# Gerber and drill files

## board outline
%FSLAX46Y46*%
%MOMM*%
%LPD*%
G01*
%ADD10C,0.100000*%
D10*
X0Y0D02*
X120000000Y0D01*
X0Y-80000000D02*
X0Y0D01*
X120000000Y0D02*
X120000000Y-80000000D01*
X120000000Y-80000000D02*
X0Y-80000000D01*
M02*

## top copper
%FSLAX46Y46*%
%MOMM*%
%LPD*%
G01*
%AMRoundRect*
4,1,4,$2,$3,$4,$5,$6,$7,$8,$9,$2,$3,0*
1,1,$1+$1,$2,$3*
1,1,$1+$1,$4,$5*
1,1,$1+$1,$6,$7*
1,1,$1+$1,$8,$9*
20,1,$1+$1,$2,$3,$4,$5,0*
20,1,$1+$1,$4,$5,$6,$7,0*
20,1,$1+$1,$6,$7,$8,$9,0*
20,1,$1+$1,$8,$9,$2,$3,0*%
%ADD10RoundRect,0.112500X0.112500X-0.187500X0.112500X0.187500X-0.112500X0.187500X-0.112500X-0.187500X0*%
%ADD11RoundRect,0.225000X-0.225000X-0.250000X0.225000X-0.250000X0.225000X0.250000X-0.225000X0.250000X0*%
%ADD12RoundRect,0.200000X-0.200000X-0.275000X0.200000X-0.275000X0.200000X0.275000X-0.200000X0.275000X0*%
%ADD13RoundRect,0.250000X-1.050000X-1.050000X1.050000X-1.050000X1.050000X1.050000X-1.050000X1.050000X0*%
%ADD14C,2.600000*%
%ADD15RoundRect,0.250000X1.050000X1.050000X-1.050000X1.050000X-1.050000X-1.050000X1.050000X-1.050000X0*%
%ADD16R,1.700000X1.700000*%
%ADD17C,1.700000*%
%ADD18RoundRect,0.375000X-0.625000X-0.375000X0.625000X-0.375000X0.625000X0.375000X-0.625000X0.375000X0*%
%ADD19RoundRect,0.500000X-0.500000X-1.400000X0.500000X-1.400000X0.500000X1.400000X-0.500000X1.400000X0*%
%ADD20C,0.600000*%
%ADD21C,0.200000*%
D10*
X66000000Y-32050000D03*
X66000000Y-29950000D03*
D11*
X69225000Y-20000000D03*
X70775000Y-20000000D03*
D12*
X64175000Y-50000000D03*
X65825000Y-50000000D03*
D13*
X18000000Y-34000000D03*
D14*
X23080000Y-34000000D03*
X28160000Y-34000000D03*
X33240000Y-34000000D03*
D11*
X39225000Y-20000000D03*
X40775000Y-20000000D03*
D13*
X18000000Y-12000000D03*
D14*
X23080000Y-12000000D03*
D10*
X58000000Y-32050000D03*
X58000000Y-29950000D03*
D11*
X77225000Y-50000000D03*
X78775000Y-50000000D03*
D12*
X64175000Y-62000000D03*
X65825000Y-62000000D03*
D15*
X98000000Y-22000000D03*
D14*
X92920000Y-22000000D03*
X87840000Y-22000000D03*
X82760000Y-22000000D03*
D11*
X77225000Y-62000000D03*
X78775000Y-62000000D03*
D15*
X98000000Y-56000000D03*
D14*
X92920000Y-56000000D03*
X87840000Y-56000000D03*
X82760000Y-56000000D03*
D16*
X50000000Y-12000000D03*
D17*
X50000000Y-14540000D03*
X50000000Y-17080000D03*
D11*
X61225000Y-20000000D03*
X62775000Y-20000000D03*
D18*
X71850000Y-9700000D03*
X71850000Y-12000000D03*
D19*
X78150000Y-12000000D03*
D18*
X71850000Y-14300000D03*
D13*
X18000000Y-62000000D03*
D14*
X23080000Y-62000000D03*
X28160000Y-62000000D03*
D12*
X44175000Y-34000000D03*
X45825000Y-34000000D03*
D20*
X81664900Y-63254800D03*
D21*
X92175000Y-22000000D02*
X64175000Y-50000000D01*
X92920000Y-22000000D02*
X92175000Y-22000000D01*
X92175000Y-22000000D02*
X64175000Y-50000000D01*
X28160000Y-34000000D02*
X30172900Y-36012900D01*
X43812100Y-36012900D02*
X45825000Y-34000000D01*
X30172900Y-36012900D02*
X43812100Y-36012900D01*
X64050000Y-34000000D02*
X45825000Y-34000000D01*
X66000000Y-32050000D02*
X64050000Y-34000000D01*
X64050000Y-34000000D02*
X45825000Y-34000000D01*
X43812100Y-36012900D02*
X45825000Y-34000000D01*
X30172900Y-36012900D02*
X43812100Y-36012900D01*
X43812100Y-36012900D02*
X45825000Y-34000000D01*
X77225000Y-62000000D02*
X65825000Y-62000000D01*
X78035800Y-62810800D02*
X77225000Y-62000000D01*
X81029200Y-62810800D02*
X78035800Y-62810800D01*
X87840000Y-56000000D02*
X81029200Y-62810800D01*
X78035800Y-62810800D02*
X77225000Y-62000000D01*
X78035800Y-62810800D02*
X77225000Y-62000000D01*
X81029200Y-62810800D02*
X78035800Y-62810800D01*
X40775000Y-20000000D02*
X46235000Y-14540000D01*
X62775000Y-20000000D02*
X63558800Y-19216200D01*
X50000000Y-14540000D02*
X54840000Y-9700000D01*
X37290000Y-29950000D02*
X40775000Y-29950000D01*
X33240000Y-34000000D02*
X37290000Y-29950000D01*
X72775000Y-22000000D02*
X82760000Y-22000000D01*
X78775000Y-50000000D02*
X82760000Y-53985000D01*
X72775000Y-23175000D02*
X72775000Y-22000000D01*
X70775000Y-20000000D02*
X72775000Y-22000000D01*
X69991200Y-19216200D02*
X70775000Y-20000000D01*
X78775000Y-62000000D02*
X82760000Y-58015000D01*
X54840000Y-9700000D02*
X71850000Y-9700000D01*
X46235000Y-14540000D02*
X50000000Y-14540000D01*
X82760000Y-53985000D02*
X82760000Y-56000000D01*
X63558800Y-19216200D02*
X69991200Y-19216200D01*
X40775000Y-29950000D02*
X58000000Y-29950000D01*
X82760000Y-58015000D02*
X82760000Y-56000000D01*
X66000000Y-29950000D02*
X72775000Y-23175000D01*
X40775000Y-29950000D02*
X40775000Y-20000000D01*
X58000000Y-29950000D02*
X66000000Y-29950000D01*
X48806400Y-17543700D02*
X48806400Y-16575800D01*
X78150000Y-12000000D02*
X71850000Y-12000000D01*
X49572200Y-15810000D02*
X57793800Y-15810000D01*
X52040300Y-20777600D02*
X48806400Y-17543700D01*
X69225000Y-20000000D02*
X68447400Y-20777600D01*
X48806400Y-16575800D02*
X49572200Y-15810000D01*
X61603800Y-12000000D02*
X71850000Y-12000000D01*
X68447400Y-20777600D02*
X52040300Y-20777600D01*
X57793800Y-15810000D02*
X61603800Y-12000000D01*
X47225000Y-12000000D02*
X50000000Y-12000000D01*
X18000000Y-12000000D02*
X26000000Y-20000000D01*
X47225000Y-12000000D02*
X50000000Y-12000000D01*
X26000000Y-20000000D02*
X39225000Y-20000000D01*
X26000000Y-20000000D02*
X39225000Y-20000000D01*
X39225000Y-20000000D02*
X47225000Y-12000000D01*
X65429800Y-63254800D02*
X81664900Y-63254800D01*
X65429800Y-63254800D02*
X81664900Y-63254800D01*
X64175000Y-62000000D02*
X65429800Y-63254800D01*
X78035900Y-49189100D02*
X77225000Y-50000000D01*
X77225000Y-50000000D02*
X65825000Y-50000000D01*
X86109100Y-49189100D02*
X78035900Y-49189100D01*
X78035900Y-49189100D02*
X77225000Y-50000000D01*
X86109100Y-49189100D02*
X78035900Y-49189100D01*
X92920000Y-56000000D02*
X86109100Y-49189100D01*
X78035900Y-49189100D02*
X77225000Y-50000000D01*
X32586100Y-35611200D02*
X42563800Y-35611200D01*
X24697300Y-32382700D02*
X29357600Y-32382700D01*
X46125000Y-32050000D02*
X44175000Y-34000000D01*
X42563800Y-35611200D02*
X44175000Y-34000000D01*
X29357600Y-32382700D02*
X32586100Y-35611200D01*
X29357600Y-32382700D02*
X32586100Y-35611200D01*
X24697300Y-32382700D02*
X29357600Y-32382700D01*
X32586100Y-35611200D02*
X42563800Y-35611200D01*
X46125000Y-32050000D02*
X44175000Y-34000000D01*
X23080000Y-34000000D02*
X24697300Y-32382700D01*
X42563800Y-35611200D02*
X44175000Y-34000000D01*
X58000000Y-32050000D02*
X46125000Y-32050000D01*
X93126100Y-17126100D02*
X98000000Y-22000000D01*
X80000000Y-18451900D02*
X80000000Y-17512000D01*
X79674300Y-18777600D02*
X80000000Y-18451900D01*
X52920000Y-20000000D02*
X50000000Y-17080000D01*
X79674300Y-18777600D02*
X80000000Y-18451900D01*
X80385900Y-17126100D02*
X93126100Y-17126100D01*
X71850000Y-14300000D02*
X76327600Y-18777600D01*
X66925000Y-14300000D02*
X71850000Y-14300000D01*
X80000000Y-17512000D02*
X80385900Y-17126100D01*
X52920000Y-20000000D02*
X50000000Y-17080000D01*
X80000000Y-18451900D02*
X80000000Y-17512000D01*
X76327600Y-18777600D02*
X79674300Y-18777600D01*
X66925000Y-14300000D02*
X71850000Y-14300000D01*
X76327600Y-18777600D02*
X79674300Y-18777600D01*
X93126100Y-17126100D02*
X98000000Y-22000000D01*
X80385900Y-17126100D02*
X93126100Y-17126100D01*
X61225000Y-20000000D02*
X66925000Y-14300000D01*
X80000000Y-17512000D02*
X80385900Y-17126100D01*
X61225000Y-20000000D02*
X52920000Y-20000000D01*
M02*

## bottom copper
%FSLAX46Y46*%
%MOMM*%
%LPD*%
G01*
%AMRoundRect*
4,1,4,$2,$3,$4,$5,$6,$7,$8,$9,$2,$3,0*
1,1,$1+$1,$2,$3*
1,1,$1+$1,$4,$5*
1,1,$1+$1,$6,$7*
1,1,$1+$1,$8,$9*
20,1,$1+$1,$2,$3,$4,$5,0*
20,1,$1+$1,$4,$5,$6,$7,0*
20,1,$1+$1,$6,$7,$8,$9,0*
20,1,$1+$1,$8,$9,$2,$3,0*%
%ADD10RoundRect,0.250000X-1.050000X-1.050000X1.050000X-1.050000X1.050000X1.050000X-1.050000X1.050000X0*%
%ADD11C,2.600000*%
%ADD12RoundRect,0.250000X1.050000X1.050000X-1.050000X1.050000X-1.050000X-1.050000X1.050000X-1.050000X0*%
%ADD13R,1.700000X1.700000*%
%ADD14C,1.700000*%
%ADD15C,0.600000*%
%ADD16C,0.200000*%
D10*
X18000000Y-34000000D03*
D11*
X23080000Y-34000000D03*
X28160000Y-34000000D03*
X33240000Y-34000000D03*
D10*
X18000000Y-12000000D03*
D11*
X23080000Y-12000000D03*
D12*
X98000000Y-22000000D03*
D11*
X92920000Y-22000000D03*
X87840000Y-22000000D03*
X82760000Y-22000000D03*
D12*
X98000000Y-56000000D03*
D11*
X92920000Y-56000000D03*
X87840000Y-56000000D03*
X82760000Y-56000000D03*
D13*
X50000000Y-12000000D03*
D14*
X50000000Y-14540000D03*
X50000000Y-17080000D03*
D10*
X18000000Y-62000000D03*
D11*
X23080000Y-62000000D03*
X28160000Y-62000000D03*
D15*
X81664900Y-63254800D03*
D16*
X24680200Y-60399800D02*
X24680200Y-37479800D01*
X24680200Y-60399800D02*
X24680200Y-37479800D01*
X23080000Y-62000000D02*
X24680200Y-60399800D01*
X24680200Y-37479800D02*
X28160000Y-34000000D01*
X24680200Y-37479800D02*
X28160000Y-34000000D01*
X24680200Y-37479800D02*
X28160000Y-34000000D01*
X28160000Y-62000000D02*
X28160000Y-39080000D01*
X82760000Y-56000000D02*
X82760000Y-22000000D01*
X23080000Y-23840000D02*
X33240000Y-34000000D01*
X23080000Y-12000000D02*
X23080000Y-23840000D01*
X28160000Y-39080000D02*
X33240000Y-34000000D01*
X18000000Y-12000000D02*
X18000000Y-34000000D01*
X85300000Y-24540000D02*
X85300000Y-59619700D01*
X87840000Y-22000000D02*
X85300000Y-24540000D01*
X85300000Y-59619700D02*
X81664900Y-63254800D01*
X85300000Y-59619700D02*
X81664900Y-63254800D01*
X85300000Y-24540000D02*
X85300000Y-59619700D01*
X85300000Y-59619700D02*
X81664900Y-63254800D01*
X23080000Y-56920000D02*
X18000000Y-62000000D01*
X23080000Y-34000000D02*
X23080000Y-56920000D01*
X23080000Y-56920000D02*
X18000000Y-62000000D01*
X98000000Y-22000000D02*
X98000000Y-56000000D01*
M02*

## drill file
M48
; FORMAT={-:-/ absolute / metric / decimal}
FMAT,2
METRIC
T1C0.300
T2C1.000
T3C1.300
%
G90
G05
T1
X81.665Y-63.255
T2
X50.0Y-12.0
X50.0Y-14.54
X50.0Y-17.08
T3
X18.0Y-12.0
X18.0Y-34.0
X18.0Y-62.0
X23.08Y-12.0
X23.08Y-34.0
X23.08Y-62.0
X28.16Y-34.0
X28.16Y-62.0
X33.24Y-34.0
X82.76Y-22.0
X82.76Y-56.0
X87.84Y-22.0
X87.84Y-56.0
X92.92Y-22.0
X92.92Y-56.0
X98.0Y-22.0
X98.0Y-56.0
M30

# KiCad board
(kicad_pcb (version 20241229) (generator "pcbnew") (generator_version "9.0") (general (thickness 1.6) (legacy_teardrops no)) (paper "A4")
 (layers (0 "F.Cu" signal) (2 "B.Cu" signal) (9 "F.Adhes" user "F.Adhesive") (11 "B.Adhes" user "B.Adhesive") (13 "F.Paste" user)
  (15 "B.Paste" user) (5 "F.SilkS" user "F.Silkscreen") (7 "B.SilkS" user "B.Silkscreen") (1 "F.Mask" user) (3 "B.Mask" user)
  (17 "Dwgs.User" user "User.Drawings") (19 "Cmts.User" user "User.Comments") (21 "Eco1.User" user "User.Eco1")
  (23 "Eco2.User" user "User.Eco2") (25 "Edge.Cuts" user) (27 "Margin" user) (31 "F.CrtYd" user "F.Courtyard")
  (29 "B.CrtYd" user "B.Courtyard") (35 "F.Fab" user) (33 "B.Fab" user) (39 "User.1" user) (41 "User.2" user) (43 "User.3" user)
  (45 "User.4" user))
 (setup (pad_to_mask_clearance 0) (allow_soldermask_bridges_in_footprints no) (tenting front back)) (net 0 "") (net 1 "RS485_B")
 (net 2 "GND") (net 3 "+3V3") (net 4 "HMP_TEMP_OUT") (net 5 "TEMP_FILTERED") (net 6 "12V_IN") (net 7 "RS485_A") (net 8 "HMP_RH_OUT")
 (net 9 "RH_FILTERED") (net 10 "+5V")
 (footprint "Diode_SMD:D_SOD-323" (layer "F.Cu") (at 66 31 90)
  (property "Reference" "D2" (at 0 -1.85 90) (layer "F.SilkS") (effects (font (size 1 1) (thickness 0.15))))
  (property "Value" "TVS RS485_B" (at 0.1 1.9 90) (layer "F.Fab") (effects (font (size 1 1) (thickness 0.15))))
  (pad "1" smd roundrect (at -1.05 0 90) (size 0.6 0.45) (layers "F.Cu" "F.Mask" "F.Paste") (roundrect_rratio 0.25) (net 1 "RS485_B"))
  (pad "2" smd roundrect (at 1.05 0 90) (size 0.6 0.45) (layers "F.Cu" "F.Mask" "F.Paste") (roundrect_rratio 0.25) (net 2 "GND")))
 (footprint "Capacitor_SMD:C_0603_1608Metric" (layer "F.Cu") (at 70 20)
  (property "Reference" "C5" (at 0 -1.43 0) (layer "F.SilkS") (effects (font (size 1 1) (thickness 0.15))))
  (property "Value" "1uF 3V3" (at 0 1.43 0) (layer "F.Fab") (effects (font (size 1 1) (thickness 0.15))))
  (pad "1" smd roundrect (at -0.775 0) (size 0.9 0.95) (layers "F.Cu" "F.Mask" "F.Paste") (roundrect_rratio 0.25) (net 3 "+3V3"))
  (pad "2" smd roundrect (at 0.775 0) (size 0.9 0.95) (layers "F.Cu" "F.Mask" "F.Paste") (roundrect_rratio 0.25) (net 2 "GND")))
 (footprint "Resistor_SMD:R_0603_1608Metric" (layer "F.Cu") (at 65 50)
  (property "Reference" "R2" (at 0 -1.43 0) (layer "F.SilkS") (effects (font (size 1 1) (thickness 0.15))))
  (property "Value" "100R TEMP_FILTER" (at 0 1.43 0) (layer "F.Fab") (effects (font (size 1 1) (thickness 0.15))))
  (pad "1" smd roundrect (at -0.825 0) (size 0.8 0.95) (layers "F.Cu" "F.Mask" "F.Paste") (roundrect_rratio 0.25) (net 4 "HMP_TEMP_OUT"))
  (pad "2" smd roundrect (at 0.825 0) (size 0.8 0.95) (layers "F.Cu" "F.Mask" "F.Paste") (roundrect_rratio 0.25) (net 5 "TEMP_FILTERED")))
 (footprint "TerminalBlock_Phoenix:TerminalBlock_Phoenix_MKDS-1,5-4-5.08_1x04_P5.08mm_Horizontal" (layer "F.Cu") (at 18 34)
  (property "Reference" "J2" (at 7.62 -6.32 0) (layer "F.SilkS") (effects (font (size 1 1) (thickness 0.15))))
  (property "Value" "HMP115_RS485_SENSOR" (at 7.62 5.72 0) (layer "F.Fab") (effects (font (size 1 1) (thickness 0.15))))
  (pad "1" thru_hole roundrect (at 0 0) (size 2.6 2.6) (drill 1.3) (layers "*.Cu" "*.Mask") (remove_unused_layers no)
   (roundrect_rratio 0.096154) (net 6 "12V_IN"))
  (pad "2" thru_hole circle (at 5.08 0) (size 2.6 2.6) (drill 1.3) (layers "*.Cu" "*.Mask") (remove_unused_layers no) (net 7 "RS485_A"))
  (pad "3" thru_hole circle (at 10.16 0) (size 2.6 2.6) (drill 1.3) (layers "*.Cu" "*.Mask") (remove_unused_layers no) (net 1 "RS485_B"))
  (pad "4" thru_hole circle (at 15.24 0) (size 2.6 2.6) (drill 1.3) (layers "*.Cu" "*.Mask") (remove_unused_layers no) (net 2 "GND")))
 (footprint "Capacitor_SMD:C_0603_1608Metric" (layer "F.Cu") (at 40 20)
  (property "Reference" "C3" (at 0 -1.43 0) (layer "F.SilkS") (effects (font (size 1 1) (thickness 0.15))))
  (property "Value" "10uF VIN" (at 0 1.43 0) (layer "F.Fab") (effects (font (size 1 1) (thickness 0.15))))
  (pad "1" smd roundrect (at -0.775 0) (size 0.9 0.95) (layers "F.Cu" "F.Mask" "F.Paste") (roundrect_rratio 0.25) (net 6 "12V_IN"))
  (pad "2" smd roundrect (at 0.775 0) (size 0.9 0.95) (layers "F.Cu" "F.Mask" "F.Paste") (roundrect_rratio 0.25) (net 2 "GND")))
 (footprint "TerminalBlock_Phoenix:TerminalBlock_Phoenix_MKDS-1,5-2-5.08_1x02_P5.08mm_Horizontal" (layer "F.Cu") (at 18 12)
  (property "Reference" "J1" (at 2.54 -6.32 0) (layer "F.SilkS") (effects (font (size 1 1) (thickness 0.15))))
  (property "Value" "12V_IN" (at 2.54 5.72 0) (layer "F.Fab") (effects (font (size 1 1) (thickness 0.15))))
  (pad "1" thru_hole roundrect (at 0 0) (size 2.6 2.6) (drill 1.3) (layers "*.Cu" "*.Mask") (remove_unused_layers no)
   (roundrect_rratio 0.096154) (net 6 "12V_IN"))
  (pad "2" thru_hole circle (at 5.08 0) (size 2.6 2.6) (drill 1.3) (layers "*.Cu" "*.Mask") (remove_unused_layers no) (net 2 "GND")))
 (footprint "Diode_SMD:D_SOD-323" (layer "F.Cu") (at 58 31 90)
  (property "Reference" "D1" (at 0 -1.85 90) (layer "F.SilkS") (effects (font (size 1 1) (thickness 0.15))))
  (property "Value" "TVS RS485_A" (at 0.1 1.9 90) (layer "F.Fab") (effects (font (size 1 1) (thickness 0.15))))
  (pad "1" smd roundrect (at -1.05 0 90) (size 0.6 0.45) (layers "F.Cu" "F.Mask" "F.Paste") (roundrect_rratio 0.25) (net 7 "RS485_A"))
  (pad "2" smd roundrect (at 1.05 0 90) (size 0.6 0.45) (layers "F.Cu" "F.Mask" "F.Paste") (roundrect_rratio 0.25) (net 2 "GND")))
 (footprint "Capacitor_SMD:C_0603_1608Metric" (layer "F.Cu") (at 78 50)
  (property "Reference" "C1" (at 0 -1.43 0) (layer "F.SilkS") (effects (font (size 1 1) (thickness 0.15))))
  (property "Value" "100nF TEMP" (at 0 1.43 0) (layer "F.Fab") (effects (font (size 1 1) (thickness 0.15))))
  (pad "1" smd roundrect (at -0.775 0) (size 0.9 0.95) (layers "F.Cu" "F.Mask" "F.Paste") (roundrect_rratio 0.25) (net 5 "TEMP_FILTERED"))
  (pad "2" smd roundrect (at 0.775 0) (size 0.9 0.95) (layers "F.Cu" "F.Mask" "F.Paste") (roundrect_rratio 0.25) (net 2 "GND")))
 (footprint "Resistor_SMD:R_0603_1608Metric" (layer "F.Cu") (at 65 62)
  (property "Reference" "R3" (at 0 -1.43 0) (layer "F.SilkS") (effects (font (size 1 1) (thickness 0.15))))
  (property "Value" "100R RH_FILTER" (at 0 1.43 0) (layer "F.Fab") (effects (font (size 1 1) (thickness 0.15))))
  (pad "1" smd roundrect (at -0.825 0) (size 0.8 0.95) (layers "F.Cu" "F.Mask" "F.Paste") (roundrect_rratio 0.25) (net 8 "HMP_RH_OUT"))
  (pad "2" smd roundrect (at 0.825 0) (size 0.8 0.95) (layers "F.Cu" "F.Mask" "F.Paste") (roundrect_rratio 0.25) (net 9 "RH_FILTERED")))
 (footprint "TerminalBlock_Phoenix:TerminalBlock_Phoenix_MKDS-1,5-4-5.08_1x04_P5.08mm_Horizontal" (layer "F.Cu") (at 98 22 180)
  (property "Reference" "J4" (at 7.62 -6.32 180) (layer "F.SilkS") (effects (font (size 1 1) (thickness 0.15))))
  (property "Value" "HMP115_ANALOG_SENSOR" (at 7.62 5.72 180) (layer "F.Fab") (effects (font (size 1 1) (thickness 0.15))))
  (pad "1" thru_hole roundrect (at 0 0 180) (size 2.6 2.6) (drill 1.3) (layers "*.Cu" "*.Mask") (remove_unused_layers no)
   (roundrect_rratio 0.096154) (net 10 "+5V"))
  (pad "2" thru_hole circle (at 5.08 0 180) (size 2.6 2.6) (drill 1.3) (layers "*.Cu" "*.Mask") (remove_unused_layers no)
   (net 4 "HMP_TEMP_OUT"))
  (pad "3" thru_hole circle (at 10.16 0 180) (size 2.6 2.6) (drill 1.3) (layers "*.Cu" "*.Mask") (remove_unused_layers no)
   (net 8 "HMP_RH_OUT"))
  (pad "4" thru_hole circle (at 15.24 0 180) (size 2.6 2.6) (drill 1.3) (layers "*.Cu" "*.Mask") (remove_unused_layers no) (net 2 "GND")))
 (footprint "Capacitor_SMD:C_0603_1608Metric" (layer "F.Cu") (at 78 62)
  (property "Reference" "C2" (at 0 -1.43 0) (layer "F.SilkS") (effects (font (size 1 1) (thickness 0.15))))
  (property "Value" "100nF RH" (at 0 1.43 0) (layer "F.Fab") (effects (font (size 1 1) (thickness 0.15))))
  (pad "1" smd roundrect (at -0.775 0) (size 0.9 0.95) (layers "F.Cu" "F.Mask" "F.Paste") (roundrect_rratio 0.25) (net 9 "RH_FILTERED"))
  (pad "2" smd roundrect (at 0.775 0) (size 0.9 0.95) (layers "F.Cu" "F.Mask" "F.Paste") (roundrect_rratio 0.25) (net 2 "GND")))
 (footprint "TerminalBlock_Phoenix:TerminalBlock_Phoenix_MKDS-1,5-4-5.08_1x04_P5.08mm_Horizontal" (layer "F.Cu") (at 98 56 180)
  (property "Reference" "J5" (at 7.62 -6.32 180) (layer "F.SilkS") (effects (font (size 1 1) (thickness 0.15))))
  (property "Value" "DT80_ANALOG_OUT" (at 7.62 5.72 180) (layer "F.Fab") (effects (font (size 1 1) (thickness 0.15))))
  (pad "1" thru_hole roundrect (at 0 0 180) (size 2.6 2.6) (drill 1.3) (layers "*.Cu" "*.Mask") (remove_unused_layers no)
   (roundrect_rratio 0.096154) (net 10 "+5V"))
  (pad "2" thru_hole circle (at 5.08 0 180) (size 2.6 2.6) (drill 1.3) (layers "*.Cu" "*.Mask") (remove_unused_layers no)
   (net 5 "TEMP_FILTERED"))
  (pad "3" thru_hole circle (at 10.16 0 180) (size 2.6 2.6) (drill 1.3) (layers "*.Cu" "*.Mask") (remove_unused_layers no)
   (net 9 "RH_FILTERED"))
  (pad "4" thru_hole circle (at 15.24 0 180) (size 2.6 2.6) (drill 1.3) (layers "*.Cu" "*.Mask") (remove_unused_layers no) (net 2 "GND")))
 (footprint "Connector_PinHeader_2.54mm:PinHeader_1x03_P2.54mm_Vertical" (layer "F.Cu") (at 50 12)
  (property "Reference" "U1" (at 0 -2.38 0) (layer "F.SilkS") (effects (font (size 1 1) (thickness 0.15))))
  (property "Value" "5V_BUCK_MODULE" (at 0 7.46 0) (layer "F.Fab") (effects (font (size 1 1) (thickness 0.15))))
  (pad "1" thru_hole rect (at 0 0) (size 1.7 1.7) (drill 1) (layers "*.Cu" "*.Mask") (remove_unused_layers no) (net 6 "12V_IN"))
  (pad "2" thru_hole circle (at 0 2.54) (size 1.7 1.7) (drill 1) (layers "*.Cu" "*.Mask") (remove_unused_layers no) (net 2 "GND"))
  (pad "3" thru_hole circle (at 0 5.08) (size 1.7 1.7) (drill 1) (layers "*.Cu" "*.Mask") (remove_unused_layers no) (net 10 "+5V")))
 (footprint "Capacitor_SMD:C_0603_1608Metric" (layer "F.Cu") (at 62 20)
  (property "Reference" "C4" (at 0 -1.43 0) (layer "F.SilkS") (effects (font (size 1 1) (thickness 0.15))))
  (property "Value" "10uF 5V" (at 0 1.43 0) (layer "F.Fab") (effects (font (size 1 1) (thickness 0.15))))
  (pad "1" smd roundrect (at -0.775 0) (size 0.9 0.95) (layers "F.Cu" "F.Mask" "F.Paste") (roundrect_rratio 0.25) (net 10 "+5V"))
  (pad "2" smd roundrect (at 0.775 0) (size 0.9 0.95) (layers "F.Cu" "F.Mask" "F.Paste") (roundrect_rratio 0.25) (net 2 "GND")))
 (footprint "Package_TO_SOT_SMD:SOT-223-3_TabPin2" (layer "F.Cu") (at 75 12)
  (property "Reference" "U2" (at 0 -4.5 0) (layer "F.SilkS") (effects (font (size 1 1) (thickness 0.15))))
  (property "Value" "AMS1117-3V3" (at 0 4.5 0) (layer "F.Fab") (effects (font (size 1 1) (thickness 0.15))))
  (pad "1" smd roundrect (at -3.15 -2.3) (size 2 1.5) (layers "F.Cu" "F.Mask" "F.Paste") (roundrect_rratio 0.25) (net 2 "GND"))
  (pad "2" smd roundrect (at -3.15 0) (size 2 1.5) (layers "F.Cu" "F.Mask" "F.Paste") (roundrect_rratio 0.25) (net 3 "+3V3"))
  (pad "2" smd roundrect (at 3.15 0) (size 2 3.8) (layers "F.Cu" "F.Mask" "F.Paste") (roundrect_rratio 0.25) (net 3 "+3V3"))
  (pad "3" smd roundrect (at -3.15 2.3) (size 2 1.5) (layers "F.Cu" "F.Mask" "F.Paste") (roundrect_rratio 0.25) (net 10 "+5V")))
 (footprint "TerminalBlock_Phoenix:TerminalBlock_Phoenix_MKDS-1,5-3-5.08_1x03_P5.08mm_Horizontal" (layer "F.Cu") (at 18 62)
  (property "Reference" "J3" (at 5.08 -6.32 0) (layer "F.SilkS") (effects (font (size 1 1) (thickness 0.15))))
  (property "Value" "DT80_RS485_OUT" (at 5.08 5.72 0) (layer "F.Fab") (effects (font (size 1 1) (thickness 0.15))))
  (pad "1" thru_hole roundrect (at 0 0) (size 2.6 2.6) (drill 1.3) (layers "*.Cu" "*.Mask") (remove_unused_layers no)
   (roundrect_rratio 0.096154) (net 7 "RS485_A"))
  (pad "2" thru_hole circle (at 5.08 0) (size 2.6 2.6) (drill 1.3) (layers "*.Cu" "*.Mask") (remove_unused_layers no) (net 1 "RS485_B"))
  (pad "3" thru_hole circle (at 10.16 0) (size 2.6 2.6) (drill 1.3) (layers "*.Cu" "*.Mask") (remove_unused_layers no) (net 2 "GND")))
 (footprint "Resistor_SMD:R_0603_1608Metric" (layer "F.Cu") (at 45 34)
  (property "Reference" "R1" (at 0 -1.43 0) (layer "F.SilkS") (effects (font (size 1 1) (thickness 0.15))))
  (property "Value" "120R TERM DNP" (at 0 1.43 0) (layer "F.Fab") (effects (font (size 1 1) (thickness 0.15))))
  (pad "1" smd roundrect (at -0.825 0) (size 0.8 0.95) (layers "F.Cu" "F.Mask" "F.Paste") (roundrect_rratio 0.25) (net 7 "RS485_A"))
  (pad "2" smd roundrect (at 0.825 0) (size 0.8 0.95) (layers "F.Cu" "F.Mask" "F.Paste") (roundrect_rratio 0.25) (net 1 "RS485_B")))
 (gr_line (start 0 0) (end 120 0) (stroke (width 0) (type default)) (layer "Edge.Cuts"))
 (gr_line (start 0 80) (end 0 0) (stroke (width 0) (type default)) (layer "Edge.Cuts"))
 (gr_line (start 120 0) (end 120 80) (stroke (width 0) (type default)) (layer "Edge.Cuts"))
 (gr_line (start 120 80) (end 0 80) (stroke (width 0) (type default)) (layer "Edge.Cuts"))
 (segment (start 92.175 22) (end 64.175 50) (width 0.2) (layer "F.Cu") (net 4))
 (segment (start 92.92 22) (end 92.175 22) (width 0.2) (layer "F.Cu") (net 4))
 (segment (start 92.175 22) (end 64.175 50) (width 0.2) (layer "F.Cu") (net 4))
 (segment (start 28.16 34) (end 30.1729 36.0129) (width 0.2) (layer "F.Cu") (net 1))
 (segment (start 43.8121 36.0129) (end 45.825 34) (width 0.2) (layer "F.Cu") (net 1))
 (segment (start 30.1729 36.0129) (end 43.8121 36.0129) (width 0.2) (layer "F.Cu") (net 1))
 (segment (start 64.05 34) (end 45.825 34) (width 0.2) (layer "F.Cu") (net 1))
 (segment (start 66 32.05) (end 64.05 34) (width 0.2) (layer "F.Cu") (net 1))
 (segment (start 64.05 34) (end 45.825 34) (width 0.2) (layer "F.Cu") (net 1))
 (segment (start 43.8121 36.0129) (end 45.825 34) (width 0.2) (layer "F.Cu") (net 1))
 (segment (start 30.1729 36.0129) (end 43.8121 36.0129) (width 0.2) (layer "F.Cu") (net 1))
 (segment (start 43.8121 36.0129) (end 45.825 34) (width 0.2) (layer "F.Cu") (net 1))
 (segment (start 24.6802 60.3998) (end 24.6802 37.4798) (width 0.2) (layer "B.Cu") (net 1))
 (segment (start 24.6802 60.3998) (end 24.6802 37.4798) (width 0.2) (layer "B.Cu") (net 1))
 (segment (start 23.08 62) (end 24.6802 60.3998) (width 0.2) (layer "B.Cu") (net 1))
 (segment (start 24.6802 37.4798) (end 28.16 34) (width 0.2) (layer "B.Cu") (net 1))
 (segment (start 24.6802 37.4798) (end 28.16 34) (width 0.2) (layer "B.Cu") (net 1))
 (segment (start 24.6802 37.4798) (end 28.16 34) (width 0.2) (layer "B.Cu") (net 1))
 (segment (start 77.225 62) (end 65.825 62) (width 0.2) (layer "F.Cu") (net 9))
 (segment (start 78.0358 62.8108) (end 77.225 62) (width 0.2) (layer "F.Cu") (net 9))
 (segment (start 81.0292 62.8108) (end 78.0358 62.8108) (width 0.2) (layer "F.Cu") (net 9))
 (segment (start 87.84 56) (end 81.0292 62.8108) (width 0.2) (layer "F.Cu") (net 9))
 (segment (start 78.0358 62.8108) (end 77.225 62) (width 0.2) (layer "F.Cu") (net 9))
 (segment (start 78.0358 62.8108) (end 77.225 62) (width 0.2) (layer "F.Cu") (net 9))
 (segment (start 81.0292 62.8108) (end 78.0358 62.8108) (width 0.2) (layer "F.Cu") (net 9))
 (segment (start 40.775 20) (end 46.235 14.54) (width 0.2) (layer "F.Cu") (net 2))
 (segment (start 62.775 20) (end 63.5588 19.2162) (width 0.2) (layer "F.Cu") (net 2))
 (segment (start 50 14.54) (end 54.84 9.7) (width 0.2) (layer "F.Cu") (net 2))
 (segment (start 37.29 29.95) (end 40.775 29.95) (width 0.2) (layer "F.Cu") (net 2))
 (segment (start 33.24 34) (end 37.29 29.95) (width 0.2) (layer "F.Cu") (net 2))
 (segment (start 72.775 22) (end 82.76 22) (width 0.2) (layer "F.Cu") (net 2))
 (segment (start 78.775 50) (end 82.76 53.985) (width 0.2) (layer "F.Cu") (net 2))
 (segment (start 72.775 23.175) (end 72.775 22) (width 0.2) (layer "F.Cu") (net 2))
 (segment (start 70.775 20) (end 72.775 22) (width 0.2) (layer "F.Cu") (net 2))
 (segment (start 69.9912 19.2162) (end 70.775 20) (width 0.2) (layer "F.Cu") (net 2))
 (segment (start 78.775 62) (end 82.76 58.015) (width 0.2) (layer "F.Cu") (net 2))
 (segment (start 54.84 9.7) (end 71.85 9.7) (width 0.2) (layer "F.Cu") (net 2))
 (segment (start 46.235 14.54) (end 50 14.54) (width 0.2) (layer "F.Cu") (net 2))
 (segment (start 82.76 53.985) (end 82.76 56) (width 0.2) (layer "F.Cu") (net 2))
 (segment (start 63.5588 19.2162) (end 69.9912 19.2162) (width 0.2) (layer "F.Cu") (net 2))
 (segment (start 40.775 29.95) (end 58 29.95) (width 0.2) (layer "F.Cu") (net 2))
 (segment (start 82.76 58.015) (end 82.76 56) (width 0.2) (layer "F.Cu") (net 2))
 (segment (start 66 29.95) (end 72.775 23.175) (width 0.2) (layer "F.Cu") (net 2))
 (segment (start 40.775 29.95) (end 40.775 20) (width 0.2) (layer "F.Cu") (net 2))
 (segment (start 58 29.95) (end 66 29.95) (width 0.2) (layer "F.Cu") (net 2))
 (segment (start 28.16 62) (end 28.16 39.08) (width 0.2) (layer "B.Cu") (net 2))
 (segment (start 82.76 56) (end 82.76 22) (width 0.2) (layer "B.Cu") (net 2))
 (segment (start 23.08 23.84) (end 33.24 34) (width 0.2) (layer "B.Cu") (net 2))
 (segment (start 23.08 12) (end 23.08 23.84) (width 0.2) (layer "B.Cu") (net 2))
 (segment (start 28.16 39.08) (end 33.24 34) (width 0.2) (layer "B.Cu") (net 2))
 (segment (start 48.8064 17.5437) (end 48.8064 16.5758) (width 0.2) (layer "F.Cu") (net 3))
 (segment (start 78.15 12) (end 71.85 12) (width 0.2) (layer "F.Cu") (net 3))
 (segment (start 49.5722 15.81) (end 57.7938 15.81) (width 0.2) (layer "F.Cu") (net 3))
 (segment (start 52.0403 20.7776) (end 48.8064 17.5437) (width 0.2) (layer "F.Cu") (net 3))
 (segment (start 69.225 20) (end 68.4474 20.7776) (width 0.2) (layer "F.Cu") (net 3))
 (segment (start 48.8064 16.5758) (end 49.5722 15.81) (width 0.2) (layer "F.Cu") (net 3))
 (segment (start 61.6038 12) (end 71.85 12) (width 0.2) (layer "F.Cu") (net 3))
 (segment (start 68.4474 20.7776) (end 52.0403 20.7776) (width 0.2) (layer "F.Cu") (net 3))
 (segment (start 57.7938 15.81) (end 61.6038 12) (width 0.2) (layer "F.Cu") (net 3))
 (segment (start 47.225 12) (end 50 12) (width 0.2) (layer "F.Cu") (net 6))
 (segment (start 18 12) (end 26 20) (width 0.2) (layer "F.Cu") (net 6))
 (segment (start 47.225 12) (end 50 12) (width 0.2) (layer "F.Cu") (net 6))
 (segment (start 26 20) (end 39.225 20) (width 0.2) (layer "F.Cu") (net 6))
 (segment (start 26 20) (end 39.225 20) (width 0.2) (layer "F.Cu") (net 6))
 (segment (start 39.225 20) (end 47.225 12) (width 0.2) (layer "F.Cu") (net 6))
 (segment (start 18 12) (end 18 34) (width 0.2) (layer "B.Cu") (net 6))
 (segment (start 65.4298 63.2548) (end 81.6649 63.2548) (width 0.2) (layer "F.Cu") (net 8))
 (segment (start 65.4298 63.2548) (end 81.6649 63.2548) (width 0.2) (layer "F.Cu") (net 8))
 (segment (start 64.175 62) (end 65.4298 63.2548) (width 0.2) (layer "F.Cu") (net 8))
 (via (at 81.6649 63.2548) (size 0.6) (drill 0.3) (layers "F.Cu" "B.Cu") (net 8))
 (segment (start 85.3 24.54) (end 85.3 59.6197) (width 0.2) (layer "B.Cu") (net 8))
 (segment (start 87.84 22) (end 85.3 24.54) (width 0.2) (layer "B.Cu") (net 8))
 (segment (start 85.3 59.6197) (end 81.6649 63.2548) (width 0.2) (layer "B.Cu") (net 8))
 (segment (start 85.3 59.6197) (end 81.6649 63.2548) (width 0.2) (layer "B.Cu") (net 8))
 (segment (start 85.3 24.54) (end 85.3 59.6197) (width 0.2) (layer "B.Cu") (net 8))
 (segment (start 85.3 59.6197) (end 81.6649 63.2548) (width 0.2) (layer "B.Cu") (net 8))
 (segment (start 78.0359 49.1891) (end 77.225 50) (width 0.2) (layer "F.Cu") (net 5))
 (segment (start 77.225 50) (end 65.825 50) (width 0.2) (layer "F.Cu") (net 5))
 (segment (start 86.1091 49.1891) (end 78.0359 49.1891) (width 0.2) (layer "F.Cu") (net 5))
 (segment (start 78.0359 49.1891) (end 77.225 50) (width 0.2) (layer "F.Cu") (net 5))
 (segment (start 86.1091 49.1891) (end 78.0359 49.1891) (width 0.2) (layer "F.Cu") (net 5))
 (segment (start 92.92 56) (end 86.1091 49.1891) (width 0.2) (layer "F.Cu") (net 5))
 (segment (start 78.0359 49.1891) (end 77.225 50) (width 0.2) (layer "F.Cu") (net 5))
 (segment (start 32.5861 35.6112) (end 42.5638 35.6112) (width 0.2) (layer "F.Cu") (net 7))
 (segment (start 24.6973 32.3827) (end 29.3576 32.3827) (width 0.2) (layer "F.Cu") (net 7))
 (segment (start 46.125 32.05) (end 44.175 34) (width 0.2) (layer "F.Cu") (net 7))
 (segment (start 42.5638 35.6112) (end 44.175 34) (width 0.2) (layer "F.Cu") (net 7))
 (segment (start 29.3576 32.3827) (end 32.5861 35.6112) (width 0.2) (layer "F.Cu") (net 7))
 (segment (start 29.3576 32.3827) (end 32.5861 35.6112) (width 0.2) (layer "F.Cu") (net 7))
 (segment (start 24.6973 32.3827) (end 29.3576 32.3827) (width 0.2) (layer "F.Cu") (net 7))
 (segment (start 32.5861 35.6112) (end 42.5638 35.6112) (width 0.2) (layer "F.Cu") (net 7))
 (segment (start 46.125 32.05) (end 44.175 34) (width 0.2) (layer "F.Cu") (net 7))
 (segment (start 23.08 34) (end 24.6973 32.3827) (width 0.2) (layer "F.Cu") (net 7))
 (segment (start 42.5638 35.6112) (end 44.175 34) (width 0.2) (layer "F.Cu") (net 7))
 (segment (start 58 32.05) (end 46.125 32.05) (width 0.2) (layer "F.Cu") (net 7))
 (segment (start 23.08 56.92) (end 18 62) (width 0.2) (layer "B.Cu") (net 7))
 (segment (start 23.08 34) (end 23.08 56.92) (width 0.2) (layer "B.Cu") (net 7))
 (segment (start 23.08 56.92) (end 18 62) (width 0.2) (layer "B.Cu") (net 7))
 (segment (start 93.1261 17.1261) (end 98 22) (width 0.2) (layer "F.Cu") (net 10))
 (segment (start 80 18.4519) (end 80 17.512) (width 0.2) (layer "F.Cu") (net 10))
 (segment (start 79.6743 18.7776) (end 80 18.4519) (width 0.2) (layer "F.Cu") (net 10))
 (segment (start 52.92 20) (end 50 17.08) (width 0.2) (layer "F.Cu") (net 10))
 (segment (start 79.6743 18.7776) (end 80 18.4519) (width 0.2) (layer "F.Cu") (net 10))
 (segment (start 80.3859 17.1261) (end 93.1261 17.1261) (width 0.2) (layer "F.Cu") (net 10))
 (segment (start 71.85 14.3) (end 76.3276 18.7776) (width 0.2) (layer "F.Cu") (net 10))
 (segment (start 66.925 14.3) (end 71.85 14.3) (width 0.2) (layer "F.Cu") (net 10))
 (segment (start 80 17.512) (end 80.3859 17.1261) (width 0.2) (layer "F.Cu") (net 10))
 (segment (start 52.92 20) (end 50 17.08) (width 0.2) (layer "F.Cu") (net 10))
 (segment (start 80 18.4519) (end 80 17.512) (width 0.2) (layer "F.Cu") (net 10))
 (segment (start 76.3276 18.7776) (end 79.6743 18.7776) (width 0.2) (layer "F.Cu") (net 10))
 (segment (start 66.925 14.3) (end 71.85 14.3) (width 0.2) (layer "F.Cu") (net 10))
 (segment (start 76.3276 18.7776) (end 79.6743 18.7776) (width 0.2) (layer "F.Cu") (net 10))
 (segment (start 93.1261 17.1261) (end 98 22) (width 0.2) (layer "F.Cu") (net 10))
 (segment (start 80.3859 17.1261) (end 93.1261 17.1261) (width 0.2) (layer "F.Cu") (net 10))
 (segment (start 61.225 20) (end 66.925 14.3) (width 0.2) (layer "F.Cu") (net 10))
 (segment (start 80 17.512) (end 80.3859 17.1261) (width 0.2) (layer "F.Cu") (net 10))
 (segment (start 61.225 20) (end 52.92 20) (width 0.2) (layer "F.Cu") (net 10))
 (segment (start 98 22) (end 98 56) (width 0.2) (layer "B.Cu") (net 10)))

